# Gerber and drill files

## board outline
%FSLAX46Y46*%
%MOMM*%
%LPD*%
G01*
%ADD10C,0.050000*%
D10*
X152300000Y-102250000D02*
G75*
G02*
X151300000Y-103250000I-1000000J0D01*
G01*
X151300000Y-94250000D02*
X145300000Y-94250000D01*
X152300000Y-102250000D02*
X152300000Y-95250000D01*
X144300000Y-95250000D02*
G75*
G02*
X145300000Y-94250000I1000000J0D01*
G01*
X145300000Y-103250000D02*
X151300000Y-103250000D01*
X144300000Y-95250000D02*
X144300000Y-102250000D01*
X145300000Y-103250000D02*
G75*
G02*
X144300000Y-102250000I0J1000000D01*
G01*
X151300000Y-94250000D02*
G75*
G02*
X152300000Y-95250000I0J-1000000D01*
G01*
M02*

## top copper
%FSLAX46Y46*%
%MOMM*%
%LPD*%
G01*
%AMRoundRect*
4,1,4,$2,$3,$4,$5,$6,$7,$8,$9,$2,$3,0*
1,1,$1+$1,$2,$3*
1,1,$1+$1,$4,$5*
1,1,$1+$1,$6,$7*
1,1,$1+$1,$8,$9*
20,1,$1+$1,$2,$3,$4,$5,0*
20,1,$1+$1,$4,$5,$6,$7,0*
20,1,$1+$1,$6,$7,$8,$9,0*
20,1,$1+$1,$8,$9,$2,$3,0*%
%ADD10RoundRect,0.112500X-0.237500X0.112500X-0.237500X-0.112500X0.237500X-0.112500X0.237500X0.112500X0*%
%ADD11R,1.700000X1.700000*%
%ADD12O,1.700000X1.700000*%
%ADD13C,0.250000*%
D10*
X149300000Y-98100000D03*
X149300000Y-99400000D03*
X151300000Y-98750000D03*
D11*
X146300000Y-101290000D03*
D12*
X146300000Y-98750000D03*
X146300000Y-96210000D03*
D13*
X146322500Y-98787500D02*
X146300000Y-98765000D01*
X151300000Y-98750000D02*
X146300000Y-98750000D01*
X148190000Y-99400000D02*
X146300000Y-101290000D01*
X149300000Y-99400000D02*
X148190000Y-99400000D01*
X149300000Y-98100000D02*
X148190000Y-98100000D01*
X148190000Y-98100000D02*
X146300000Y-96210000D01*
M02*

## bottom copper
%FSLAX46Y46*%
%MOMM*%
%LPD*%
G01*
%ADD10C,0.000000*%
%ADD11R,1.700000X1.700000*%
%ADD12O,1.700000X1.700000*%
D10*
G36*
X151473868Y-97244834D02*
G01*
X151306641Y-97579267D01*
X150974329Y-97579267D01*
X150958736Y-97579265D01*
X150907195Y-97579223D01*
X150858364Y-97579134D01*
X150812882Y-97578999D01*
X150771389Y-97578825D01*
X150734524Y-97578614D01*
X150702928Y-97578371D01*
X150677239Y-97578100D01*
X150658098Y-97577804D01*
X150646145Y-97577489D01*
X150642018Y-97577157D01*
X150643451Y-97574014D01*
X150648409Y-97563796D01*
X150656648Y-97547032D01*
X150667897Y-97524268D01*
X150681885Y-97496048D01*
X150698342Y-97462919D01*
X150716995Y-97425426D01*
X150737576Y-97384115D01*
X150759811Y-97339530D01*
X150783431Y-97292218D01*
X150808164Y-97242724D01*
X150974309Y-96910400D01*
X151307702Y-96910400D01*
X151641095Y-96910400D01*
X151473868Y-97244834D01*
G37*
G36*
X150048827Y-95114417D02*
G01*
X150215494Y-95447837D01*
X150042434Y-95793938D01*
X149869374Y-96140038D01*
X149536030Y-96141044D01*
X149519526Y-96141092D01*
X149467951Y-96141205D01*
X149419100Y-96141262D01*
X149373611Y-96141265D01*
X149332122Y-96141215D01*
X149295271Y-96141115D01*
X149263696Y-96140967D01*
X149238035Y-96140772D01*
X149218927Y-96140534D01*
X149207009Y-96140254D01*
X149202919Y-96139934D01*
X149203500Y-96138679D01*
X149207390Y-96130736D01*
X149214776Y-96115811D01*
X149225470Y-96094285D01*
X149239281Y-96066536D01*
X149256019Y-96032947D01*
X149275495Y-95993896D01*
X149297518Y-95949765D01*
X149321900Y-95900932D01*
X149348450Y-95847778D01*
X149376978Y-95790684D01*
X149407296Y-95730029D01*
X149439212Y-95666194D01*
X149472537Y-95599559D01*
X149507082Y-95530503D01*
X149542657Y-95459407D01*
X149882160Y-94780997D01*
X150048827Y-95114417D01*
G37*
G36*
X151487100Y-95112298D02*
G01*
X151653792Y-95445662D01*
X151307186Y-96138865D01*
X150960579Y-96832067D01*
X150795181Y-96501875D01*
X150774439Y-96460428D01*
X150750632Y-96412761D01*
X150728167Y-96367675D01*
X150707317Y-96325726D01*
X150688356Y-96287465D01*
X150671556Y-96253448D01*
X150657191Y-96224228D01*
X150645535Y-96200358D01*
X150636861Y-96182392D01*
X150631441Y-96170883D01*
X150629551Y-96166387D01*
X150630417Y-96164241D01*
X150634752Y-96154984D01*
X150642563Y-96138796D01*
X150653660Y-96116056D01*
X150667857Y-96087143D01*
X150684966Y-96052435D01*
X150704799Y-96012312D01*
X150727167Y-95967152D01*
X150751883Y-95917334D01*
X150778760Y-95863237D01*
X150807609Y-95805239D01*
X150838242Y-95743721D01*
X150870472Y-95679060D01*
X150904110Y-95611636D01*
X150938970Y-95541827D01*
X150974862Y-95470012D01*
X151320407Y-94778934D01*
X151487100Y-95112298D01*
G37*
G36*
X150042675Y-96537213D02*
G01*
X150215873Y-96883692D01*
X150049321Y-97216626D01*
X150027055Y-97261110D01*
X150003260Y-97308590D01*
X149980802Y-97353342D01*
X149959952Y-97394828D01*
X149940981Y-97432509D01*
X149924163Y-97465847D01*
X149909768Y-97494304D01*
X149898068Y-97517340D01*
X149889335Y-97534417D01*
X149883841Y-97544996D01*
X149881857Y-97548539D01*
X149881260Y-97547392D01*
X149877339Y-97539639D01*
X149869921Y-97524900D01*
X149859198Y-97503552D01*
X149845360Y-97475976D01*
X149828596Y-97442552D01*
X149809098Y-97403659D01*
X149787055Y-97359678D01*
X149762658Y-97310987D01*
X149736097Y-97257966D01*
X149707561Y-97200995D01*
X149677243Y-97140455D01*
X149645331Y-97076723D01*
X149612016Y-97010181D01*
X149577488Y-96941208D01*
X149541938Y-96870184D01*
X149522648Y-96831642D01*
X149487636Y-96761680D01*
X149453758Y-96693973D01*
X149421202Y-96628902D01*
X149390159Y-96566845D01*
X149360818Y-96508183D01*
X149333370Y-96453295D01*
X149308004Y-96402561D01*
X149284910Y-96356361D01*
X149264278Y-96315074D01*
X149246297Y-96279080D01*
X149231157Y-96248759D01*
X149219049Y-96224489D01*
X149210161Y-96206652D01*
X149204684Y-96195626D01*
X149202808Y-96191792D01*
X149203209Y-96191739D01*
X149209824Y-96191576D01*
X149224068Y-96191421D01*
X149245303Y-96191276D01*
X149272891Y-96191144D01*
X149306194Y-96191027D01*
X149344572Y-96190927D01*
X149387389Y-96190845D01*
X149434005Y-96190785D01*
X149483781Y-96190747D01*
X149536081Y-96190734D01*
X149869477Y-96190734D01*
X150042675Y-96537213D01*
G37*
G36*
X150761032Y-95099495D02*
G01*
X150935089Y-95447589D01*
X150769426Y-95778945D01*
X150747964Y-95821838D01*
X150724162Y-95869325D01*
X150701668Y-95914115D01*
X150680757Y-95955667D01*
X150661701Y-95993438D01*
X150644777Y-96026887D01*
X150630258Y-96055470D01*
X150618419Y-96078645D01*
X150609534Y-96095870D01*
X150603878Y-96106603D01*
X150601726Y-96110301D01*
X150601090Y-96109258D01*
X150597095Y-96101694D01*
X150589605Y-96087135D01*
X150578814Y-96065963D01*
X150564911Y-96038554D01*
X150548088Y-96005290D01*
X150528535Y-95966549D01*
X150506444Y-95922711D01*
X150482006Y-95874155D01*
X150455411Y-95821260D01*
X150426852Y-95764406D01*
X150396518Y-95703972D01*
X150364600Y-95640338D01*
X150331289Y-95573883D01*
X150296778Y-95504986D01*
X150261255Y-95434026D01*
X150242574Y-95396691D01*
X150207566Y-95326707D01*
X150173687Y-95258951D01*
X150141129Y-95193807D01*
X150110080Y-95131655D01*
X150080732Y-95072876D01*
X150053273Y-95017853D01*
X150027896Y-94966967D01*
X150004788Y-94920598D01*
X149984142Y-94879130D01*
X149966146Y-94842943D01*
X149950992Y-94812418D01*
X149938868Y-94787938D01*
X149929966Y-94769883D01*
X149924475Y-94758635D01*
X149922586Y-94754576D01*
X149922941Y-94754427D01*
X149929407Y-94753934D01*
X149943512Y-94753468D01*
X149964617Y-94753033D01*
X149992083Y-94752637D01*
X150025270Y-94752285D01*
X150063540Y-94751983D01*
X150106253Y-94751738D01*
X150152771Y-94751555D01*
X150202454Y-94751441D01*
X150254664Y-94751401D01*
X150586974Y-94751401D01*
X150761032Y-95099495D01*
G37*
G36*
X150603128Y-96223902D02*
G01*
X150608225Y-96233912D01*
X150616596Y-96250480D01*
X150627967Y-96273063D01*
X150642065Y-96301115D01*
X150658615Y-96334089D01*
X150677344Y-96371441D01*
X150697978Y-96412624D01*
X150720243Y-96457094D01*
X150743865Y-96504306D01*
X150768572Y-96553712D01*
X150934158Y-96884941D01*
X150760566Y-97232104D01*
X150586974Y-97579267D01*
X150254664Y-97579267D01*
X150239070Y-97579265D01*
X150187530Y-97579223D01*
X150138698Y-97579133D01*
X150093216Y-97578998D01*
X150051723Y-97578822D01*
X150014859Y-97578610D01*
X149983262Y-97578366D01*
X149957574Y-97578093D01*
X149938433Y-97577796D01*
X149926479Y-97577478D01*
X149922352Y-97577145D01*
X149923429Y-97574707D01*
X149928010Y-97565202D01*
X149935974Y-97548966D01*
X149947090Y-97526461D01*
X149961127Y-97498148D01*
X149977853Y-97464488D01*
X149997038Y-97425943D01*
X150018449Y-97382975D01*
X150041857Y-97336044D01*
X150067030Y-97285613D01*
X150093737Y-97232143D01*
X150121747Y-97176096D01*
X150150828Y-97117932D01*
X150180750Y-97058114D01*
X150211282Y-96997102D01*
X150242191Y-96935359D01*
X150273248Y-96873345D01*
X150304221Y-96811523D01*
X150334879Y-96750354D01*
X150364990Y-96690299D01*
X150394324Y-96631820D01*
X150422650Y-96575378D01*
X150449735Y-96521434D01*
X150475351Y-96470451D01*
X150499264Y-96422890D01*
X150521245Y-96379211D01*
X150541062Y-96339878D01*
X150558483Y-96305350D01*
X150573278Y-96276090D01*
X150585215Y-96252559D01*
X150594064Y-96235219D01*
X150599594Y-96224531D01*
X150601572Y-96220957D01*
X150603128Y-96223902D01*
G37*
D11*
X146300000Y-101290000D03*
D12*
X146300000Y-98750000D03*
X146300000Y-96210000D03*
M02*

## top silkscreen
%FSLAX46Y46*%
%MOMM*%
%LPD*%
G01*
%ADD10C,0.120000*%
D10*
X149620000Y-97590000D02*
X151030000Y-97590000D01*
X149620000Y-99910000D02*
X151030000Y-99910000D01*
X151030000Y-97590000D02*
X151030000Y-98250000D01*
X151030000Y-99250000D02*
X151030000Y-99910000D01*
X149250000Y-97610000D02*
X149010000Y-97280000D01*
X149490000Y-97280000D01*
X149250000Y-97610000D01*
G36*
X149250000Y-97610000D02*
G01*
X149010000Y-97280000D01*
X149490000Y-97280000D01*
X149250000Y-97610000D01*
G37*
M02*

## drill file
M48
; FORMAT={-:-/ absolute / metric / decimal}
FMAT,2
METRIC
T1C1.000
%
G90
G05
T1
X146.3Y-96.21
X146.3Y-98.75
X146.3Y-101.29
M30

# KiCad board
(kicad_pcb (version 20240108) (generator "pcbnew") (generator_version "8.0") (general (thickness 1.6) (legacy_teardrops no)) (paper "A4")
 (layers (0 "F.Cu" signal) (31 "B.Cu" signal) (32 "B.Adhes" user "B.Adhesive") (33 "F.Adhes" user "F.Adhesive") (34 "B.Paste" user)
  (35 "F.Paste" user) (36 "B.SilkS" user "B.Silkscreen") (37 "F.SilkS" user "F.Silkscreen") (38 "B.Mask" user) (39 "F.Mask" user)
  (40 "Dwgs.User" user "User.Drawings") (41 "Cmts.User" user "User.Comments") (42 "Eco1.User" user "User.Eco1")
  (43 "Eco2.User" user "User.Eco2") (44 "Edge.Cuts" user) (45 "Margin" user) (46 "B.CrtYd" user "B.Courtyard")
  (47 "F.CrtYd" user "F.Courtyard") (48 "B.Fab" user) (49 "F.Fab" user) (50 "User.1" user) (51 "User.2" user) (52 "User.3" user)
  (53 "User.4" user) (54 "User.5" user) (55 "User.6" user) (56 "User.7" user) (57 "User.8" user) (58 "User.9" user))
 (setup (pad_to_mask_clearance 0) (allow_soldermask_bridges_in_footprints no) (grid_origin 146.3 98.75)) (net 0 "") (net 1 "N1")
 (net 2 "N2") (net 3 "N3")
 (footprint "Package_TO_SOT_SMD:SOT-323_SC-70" (layer "F.Cu") (at 150.3 98.75)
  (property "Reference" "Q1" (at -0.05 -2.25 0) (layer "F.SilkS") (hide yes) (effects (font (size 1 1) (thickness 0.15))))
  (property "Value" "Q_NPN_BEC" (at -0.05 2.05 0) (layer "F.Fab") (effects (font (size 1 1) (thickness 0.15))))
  (fp_line (start -0.68 -1.16) (end 0.73 -1.16) (stroke (width 0.12) (type solid)) (layer "F.SilkS"))
  (fp_line (start -0.68 1.16) (end 0.73 1.16) (stroke (width 0.12) (type solid)) (layer "F.SilkS"))
  (fp_line (start 0.73 -1.16) (end 0.73 -0.5) (stroke (width 0.12) (type solid)) (layer "F.SilkS"))
  (fp_line (start 0.73 0.5) (end 0.73 1.16) (stroke (width 0.12) (type solid)) (layer "F.SilkS"))
  (fp_poly
   (pts (xy -1.05 -1.14) (xy -1.29 -1.47) (xy -0.81 -1.47) (xy -1.05 -1.14)) (stroke (width 0.12) (type solid)) (fill solid)
   (layer "F.SilkS"))
  (pad "1" smd roundrect (at -1 -0.65 270) (size 0.45 0.7) (layers "F.Cu" "F.Paste" "F.Mask") (roundrect_rratio 0.25) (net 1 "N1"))
  (pad "2" smd roundrect (at -1 0.65 270) (size 0.45 0.7) (layers "F.Cu" "F.Paste" "F.Mask") (roundrect_rratio 0.25) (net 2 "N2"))
  (pad "3" smd roundrect (at 1 0 270) (size 0.45 0.7) (layers "F.Cu" "F.Paste" "F.Mask") (roundrect_rratio 0.25) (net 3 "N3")))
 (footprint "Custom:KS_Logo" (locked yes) (layer "B.Cu") (at 150.3 96.25 90)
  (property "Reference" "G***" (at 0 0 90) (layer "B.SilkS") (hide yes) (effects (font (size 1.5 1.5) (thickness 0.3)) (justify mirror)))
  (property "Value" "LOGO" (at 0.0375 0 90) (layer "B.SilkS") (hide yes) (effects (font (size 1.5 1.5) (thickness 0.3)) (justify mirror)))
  (fp_poly
   (pts (xy -0.6604 1.007702) (xy -0.6604 0.674309) (xy -0.992724 0.508164) (xy -1.042218 0.483431) (xy -1.08953 0.459811)
    (xy -1.134115 0.437576) (xy -1.175426 0.416995) (xy -1.212919 0.398342) (xy -1.246048 0.381885) (xy -1.274268 0.367897)
    (xy -1.297032 0.356648) (xy -1.313796 0.348409) (xy -1.324014 0.343451) (xy -1.327157 0.342018) (xy -1.327489 0.346145)
    (xy -1.327804 0.358098) (xy -1.3281 0.377239) (xy -1.328371 0.402928) (xy -1.328614 0.434524) (xy -1.328825 0.471389)
    (xy -1.328999 0.512882) (xy -1.329134 0.558364) (xy -1.329223 0.607195) (xy -1.329265 0.658736) (xy -1.329267 0.674329)
    (xy -1.329267 1.006641) (xy -0.994834 1.173868) (xy -0.6604 1.341095))
   (stroke (width 0) (type solid)) (fill solid) (layer "B.Cu"))
  (fp_poly
   (pts (xy 1.135583 -0.251173) (xy 1.469003 -0.41784) (xy 0.790593 -0.757343) (xy 0.719497 -0.792918) (xy 0.650441 -0.827463)
    (xy 0.583806 -0.860788) (xy 0.519971 -0.892704) (xy 0.459316 -0.923022) (xy 0.402222 -0.95155) (xy 0.349068 -0.9781)
    (xy 0.300235 -1.002482) (xy 0.256104 -1.024505) (xy 0.217053 -1.043981) (xy 0.183464 -1.060719) (xy 0.155715 -1.07453)
    (xy 0.134189 -1.085224) (xy 0.119264 -1.09261) (xy 0.111321 -1.0965) (xy 0.110066 -1.097081) (xy 0.109746 -1.092991)
    (xy 0.109466 -1.081073) (xy 0.109228 -1.061965) (xy 0.109033 -1.036304) (xy 0.108885 -1.004729) (xy 0.108785 -0.967878)
    (xy 0.108735 -0.926389) (xy 0.108738 -0.8809) (xy 0.108795 -0.832049) (xy 0.108908 -0.780474) (xy 0.108956 -0.76397)
    (xy 0.109962 -0.430626) (xy 0.456062 -0.257566) (xy 0.802163 -0.084506))
   (stroke (width 0) (type solid)) (fill solid) (layer "B.Cu"))
  (fp_poly
   (pts (xy 1.137702 1.1871) (xy 1.471066 1.020407) (xy 0.779988 0.674862) (xy 0.708173 0.63897) (xy 0.638364 0.60411) (xy 0.57094 0.570472)
    (xy 0.506279 0.538242) (xy 0.444761 0.507609) (xy 0.386763 0.47876) (xy 0.332666 0.451883) (xy 0.282848 0.427167) (xy 0.237688 0.404799)
    (xy 0.197565 0.384966) (xy 0.162857 0.367857) (xy 0.133944 0.35366) (xy 0.111204 0.342563) (xy 0.095016 0.334752) (xy 0.085759 0.330417)
    (xy 0.083613 0.329551) (xy 0.079117 0.331441) (xy 0.067608 0.336861) (xy 0.049642 0.345535) (xy 0.025772 0.357191)
    (xy -0.003448 0.371556) (xy -0.037465 0.388356) (xy -0.075726 0.407317) (xy -0.117675 0.428167) (xy -0.162761 0.450632)
    (xy -0.210428 0.474439) (xy -0.251875 0.495181) (xy -0.582067 0.660579) (xy 0.111135 1.007186) (xy 0.804338 1.353792))
   (stroke (width 0) (type solid)) (fill solid) (layer "B.Cu"))
  (fp_poly
   (pts (xy -0.287213 -0.257325) (xy 0.059266 -0.430523) (xy 0.059266 -0.763919) (xy 0.059253 -0.816219) (xy 0.059215 -0.865995)
    (xy 0.059155 -0.912611) (xy 0.059073 -0.955428) (xy 0.058973 -0.993806) (xy 0.058856 -1.027109) (xy 0.058724 -1.054697)
    (xy 0.058579 -1.075932) (xy 0.058424 -1.090176) (xy 0.058261 -1.096791) (xy 0.058208 -1.097192) (xy 0.054374 -1.095316)
    (xy 0.043348 -1.089839) (xy 0.025511 -1.080951) (xy 0.001241 -1.068843) (xy -0.02908 -1.053703) (xy -0.065074 -1.035722)
    (xy -0.106361 -1.01509) (xy -0.152561 -0.991996) (xy -0.203295 -0.96663) (xy -0.258183 -0.939182) (xy -0.316845 -0.909841)
    (xy -0.378902 -0.878798) (xy -0.443973 -0.846242) (xy -0.51168 -0.812364) (xy -0.581642 -0.777352) (xy -0.620184 -0.758062)
    (xy -0.691208 -0.722512) (xy -0.760181 -0.687984) (xy -0.826723 -0.654669) (xy -0.890455 -0.622757) (xy -0.950995 -0.592439)
    (xy -1.007966 -0.563903) (xy -1.060987 -0.537342) (xy -1.109678 -0.512945) (xy -1.153659 -0.490902) (xy -1.192552 -0.471404)
    (xy -1.225976 -0.45464) (xy -1.253552 -0.440802) (xy -1.2749 -0.430079) (xy -1.289639 -0.422661) (xy -1.297392 -0.41874)
    (xy -1.298539 -0.418143) (xy -1.294996 -0.416159) (xy -1.284417 -0.410665) (xy -1.26734 -0.401932) (xy -1.244304 -0.390232)
    (xy -1.215847 -0.375837) (xy -1.182509 -0.359019) (xy -1.144828 -0.340048) (xy -1.103342 -0.319198) (xy -1.05859 -0.29674)
    (xy -1.01111 -0.272945) (xy -0.966626 -0.250679) (xy -0.633692 -0.084127))
   (stroke (width 0) (type solid)) (fill solid) (layer "B.Cu"))
  (fp_poly
   (pts (xy 1.150505 0.461032) (xy 1.498599 0.286974) (xy 1.498599 -0.045336) (xy 1.498559 -0.097546) (xy 1.498445 -0.147229)
    (xy 1.498262 -0.193747) (xy 1.498017 -0.23646) (xy 1.497715 -0.27473) (xy 1.497363 -0.307917) (xy 1.496967 -0.335383)
    (xy 1.496532 -0.356488) (xy 1.496066 -0.370593) (xy 1.495573 -0.377059) (xy 1.495424 -0.377414) (xy 1.491365 -0.375525)
    (xy 1.480117 -0.370034) (xy 1.462062 -0.361132) (xy 1.437582 -0.349008) (xy 1.407057 -0.333854) (xy 1.37087 -0.315858)
    (xy 1.329402 -0.295212) (xy 1.283033 -0.272104) (xy 1.232147 -0.246727) (xy 1.177124 -0.219268) (xy 1.118345 -0.18992)
    (xy 1.056193 -0.158871) (xy 0.991049 -0.126313) (xy 0.923293 -0.092434) (xy 0.853309 -0.057426) (xy 0.815974 -0.038745)
    (xy 0.745014 -0.003222) (xy 0.676117 0.031289) (xy 0.609662 0.0646) (xy 0.546028 0.096518) (xy 0.485594 0.126852) (xy 0.42874 0.155411)
    (xy 0.375845 0.182006) (xy 0.327289 0.206444) (xy 0.283451 0.228535) (xy 0.24471 0.248088) (xy 0.211446 0.264911) (xy 0.184037 0.278814)
    (xy 0.162865 0.289605) (xy 0.148306 0.297095) (xy 0.140742 0.30109) (xy 0.139699 0.301726) (xy 0.143397 0.303878) (xy 0.15413 0.309534)
    (xy 0.171355 0.318419) (xy 0.19453 0.330258) (xy 0.223113 0.344777) (xy 0.256562 0.361701) (xy 0.294333 0.380757) (xy 0.335885 0.401668)
    (xy 0.380675 0.424162) (xy 0.428162 0.447964) (xy 0.471055 0.469426) (xy 0.802411 0.635089))
   (stroke (width 0) (type solid)) (fill solid) (layer "B.Cu"))
  (fp_poly
   (pts (xy -0.303712 0.468572) (xy -0.254306 0.443865) (xy -0.207094 0.420243) (xy -0.162624 0.397978) (xy -0.121441 0.377344)
    (xy -0.084089 0.358615) (xy -0.051115 0.342065) (xy -0.023063 0.327967) (xy -0.00048 0.316596) (xy 0.016088 0.308225)
    (xy 0.026098 0.303128) (xy 0.029043 0.301572) (xy 0.025469 0.299594) (xy 0.014781 0.294064) (xy -0.002559 0.285215)
    (xy -0.02609 0.273278) (xy -0.05535 0.258483) (xy -0.089878 0.241062) (xy -0.129211 0.221245) (xy -0.17289 0.199264)
    (xy -0.220451 0.175351) (xy -0.271434 0.149735) (xy -0.325378 0.12265) (xy -0.38182 0.094324) (xy -0.440299 0.06499)
    (xy -0.500354 0.034879) (xy -0.561523 0.004221) (xy -0.623345 -0.026752) (xy -0.685359 -0.057809) (xy -0.747102 -0.088718)
    (xy -0.808114 -0.11925) (xy -0.867932 -0.149172) (xy -0.926096 -0.178253) (xy -0.982143 -0.206263) (xy -1.035613 -0.23297)
    (xy -1.086044 -0.258143) (xy -1.132975 -0.281551) (xy -1.175943 -0.302962) (xy -1.214488 -0.322147) (xy -1.248148 -0.338873)
    (xy -1.276461 -0.35291) (xy -1.298966 -0.364026) (xy -1.315202 -0.37199) (xy -1.324707 -0.376571) (xy -1.327145 -0.377648)
    (xy -1.327478 -0.373521) (xy -1.327796 -0.361567) (xy -1.328093 -0.342426) (xy -1.328366 -0.316738) (xy -1.32861 -0.285141)
    (xy -1.328822 -0.248277) (xy -1.328998 -0.206784) (xy -1.329133 -0.161302) (xy -1.329223 -0.11247) (xy -1.329265 -0.06093)
    (xy -1.329267 -0.045336) (xy -1.329267 0.286974) (xy -0.982104 0.460566) (xy -0.634941 0.634158))
   (stroke (width 0) (type solid)) (fill solid) (layer "B.Cu")))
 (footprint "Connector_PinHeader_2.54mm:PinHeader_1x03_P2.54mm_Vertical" (layer "B.Cu") (at 146.3 101.29)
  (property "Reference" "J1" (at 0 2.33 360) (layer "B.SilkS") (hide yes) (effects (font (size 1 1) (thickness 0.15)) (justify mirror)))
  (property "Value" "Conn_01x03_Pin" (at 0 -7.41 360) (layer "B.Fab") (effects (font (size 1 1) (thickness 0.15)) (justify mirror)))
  (pad "1" thru_hole rect (at 0 0) (size 1.7 1.7) (drill 1) (layers "*.Cu" "*.Mask") (remove_unused_layers no) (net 2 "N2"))
  (pad "2" thru_hole oval (at 0 -2.54) (size 1.7 1.7) (drill 1) (layers "*.Cu" "*.Mask") (remove_unused_layers no) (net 3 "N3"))
  (pad "3" thru_hole oval (at 0 -5.08) (size 1.7 1.7) (drill 1) (layers "*.Cu" "*.Mask") (remove_unused_layers no) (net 1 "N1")))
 (gr_arc (start 152.3 102.25) (mid 152.007107 102.957107) (end 151.3 103.25) (stroke (width 0.05) (type default)) (layer "Edge.Cuts"))
 (gr_line (start 151.3 94.25) (end 145.3 94.25) (stroke (width 0.05) (type default)) (layer "Edge.Cuts"))
 (gr_line (start 152.3 102.25) (end 152.3 95.25) (stroke (width 0.05) (type default)) (layer "Edge.Cuts"))
 (gr_arc (start 144.3 95.25) (mid 144.592893 94.542893) (end 145.3 94.25) (stroke (width 0.05) (type default)) (layer "Edge.Cuts"))
 (gr_line (start 145.3 103.25) (end 151.3 103.25) (stroke (width 0.05) (type default)) (layer "Edge.Cuts"))
 (gr_line (start 144.3 95.25) (end 144.3 102.25) (stroke (width 0.05) (type default)) (layer "Edge.Cuts"))
 (gr_arc (start 145.3 103.25) (mid 144.592893 102.957107) (end 144.3 102.25) (stroke (width 0.05) (type default)) (layer "Edge.Cuts"))
 (gr_arc (start 151.3 94.25) (mid 152.007107 94.542893) (end 152.3 95.25) (stroke (width 0.05) (type default)) (layer "Edge.Cuts"))
 (segment (start 146.3225 98.7875) (end 146.3 98.765) (width 0.25) (layer "F.Cu") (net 3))
 (segment (start 151.3 98.75) (end 146.3 98.75) (width 0.25) (layer "F.Cu") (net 3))
 (segment (start 148.19 99.4) (end 146.3 101.29) (width 0.25) (layer "F.Cu") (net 2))
 (segment (start 149.3 99.4) (end 148.19 99.4) (width 0.25) (layer "F.Cu") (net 2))
 (segment (start 149.3 98.1) (end 148.19 98.1) (width 0.25) (layer "F.Cu") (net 1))
 (segment (start 148.19 98.1) (end 146.3 96.21) (width 0.25) (layer "F.Cu") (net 1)))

